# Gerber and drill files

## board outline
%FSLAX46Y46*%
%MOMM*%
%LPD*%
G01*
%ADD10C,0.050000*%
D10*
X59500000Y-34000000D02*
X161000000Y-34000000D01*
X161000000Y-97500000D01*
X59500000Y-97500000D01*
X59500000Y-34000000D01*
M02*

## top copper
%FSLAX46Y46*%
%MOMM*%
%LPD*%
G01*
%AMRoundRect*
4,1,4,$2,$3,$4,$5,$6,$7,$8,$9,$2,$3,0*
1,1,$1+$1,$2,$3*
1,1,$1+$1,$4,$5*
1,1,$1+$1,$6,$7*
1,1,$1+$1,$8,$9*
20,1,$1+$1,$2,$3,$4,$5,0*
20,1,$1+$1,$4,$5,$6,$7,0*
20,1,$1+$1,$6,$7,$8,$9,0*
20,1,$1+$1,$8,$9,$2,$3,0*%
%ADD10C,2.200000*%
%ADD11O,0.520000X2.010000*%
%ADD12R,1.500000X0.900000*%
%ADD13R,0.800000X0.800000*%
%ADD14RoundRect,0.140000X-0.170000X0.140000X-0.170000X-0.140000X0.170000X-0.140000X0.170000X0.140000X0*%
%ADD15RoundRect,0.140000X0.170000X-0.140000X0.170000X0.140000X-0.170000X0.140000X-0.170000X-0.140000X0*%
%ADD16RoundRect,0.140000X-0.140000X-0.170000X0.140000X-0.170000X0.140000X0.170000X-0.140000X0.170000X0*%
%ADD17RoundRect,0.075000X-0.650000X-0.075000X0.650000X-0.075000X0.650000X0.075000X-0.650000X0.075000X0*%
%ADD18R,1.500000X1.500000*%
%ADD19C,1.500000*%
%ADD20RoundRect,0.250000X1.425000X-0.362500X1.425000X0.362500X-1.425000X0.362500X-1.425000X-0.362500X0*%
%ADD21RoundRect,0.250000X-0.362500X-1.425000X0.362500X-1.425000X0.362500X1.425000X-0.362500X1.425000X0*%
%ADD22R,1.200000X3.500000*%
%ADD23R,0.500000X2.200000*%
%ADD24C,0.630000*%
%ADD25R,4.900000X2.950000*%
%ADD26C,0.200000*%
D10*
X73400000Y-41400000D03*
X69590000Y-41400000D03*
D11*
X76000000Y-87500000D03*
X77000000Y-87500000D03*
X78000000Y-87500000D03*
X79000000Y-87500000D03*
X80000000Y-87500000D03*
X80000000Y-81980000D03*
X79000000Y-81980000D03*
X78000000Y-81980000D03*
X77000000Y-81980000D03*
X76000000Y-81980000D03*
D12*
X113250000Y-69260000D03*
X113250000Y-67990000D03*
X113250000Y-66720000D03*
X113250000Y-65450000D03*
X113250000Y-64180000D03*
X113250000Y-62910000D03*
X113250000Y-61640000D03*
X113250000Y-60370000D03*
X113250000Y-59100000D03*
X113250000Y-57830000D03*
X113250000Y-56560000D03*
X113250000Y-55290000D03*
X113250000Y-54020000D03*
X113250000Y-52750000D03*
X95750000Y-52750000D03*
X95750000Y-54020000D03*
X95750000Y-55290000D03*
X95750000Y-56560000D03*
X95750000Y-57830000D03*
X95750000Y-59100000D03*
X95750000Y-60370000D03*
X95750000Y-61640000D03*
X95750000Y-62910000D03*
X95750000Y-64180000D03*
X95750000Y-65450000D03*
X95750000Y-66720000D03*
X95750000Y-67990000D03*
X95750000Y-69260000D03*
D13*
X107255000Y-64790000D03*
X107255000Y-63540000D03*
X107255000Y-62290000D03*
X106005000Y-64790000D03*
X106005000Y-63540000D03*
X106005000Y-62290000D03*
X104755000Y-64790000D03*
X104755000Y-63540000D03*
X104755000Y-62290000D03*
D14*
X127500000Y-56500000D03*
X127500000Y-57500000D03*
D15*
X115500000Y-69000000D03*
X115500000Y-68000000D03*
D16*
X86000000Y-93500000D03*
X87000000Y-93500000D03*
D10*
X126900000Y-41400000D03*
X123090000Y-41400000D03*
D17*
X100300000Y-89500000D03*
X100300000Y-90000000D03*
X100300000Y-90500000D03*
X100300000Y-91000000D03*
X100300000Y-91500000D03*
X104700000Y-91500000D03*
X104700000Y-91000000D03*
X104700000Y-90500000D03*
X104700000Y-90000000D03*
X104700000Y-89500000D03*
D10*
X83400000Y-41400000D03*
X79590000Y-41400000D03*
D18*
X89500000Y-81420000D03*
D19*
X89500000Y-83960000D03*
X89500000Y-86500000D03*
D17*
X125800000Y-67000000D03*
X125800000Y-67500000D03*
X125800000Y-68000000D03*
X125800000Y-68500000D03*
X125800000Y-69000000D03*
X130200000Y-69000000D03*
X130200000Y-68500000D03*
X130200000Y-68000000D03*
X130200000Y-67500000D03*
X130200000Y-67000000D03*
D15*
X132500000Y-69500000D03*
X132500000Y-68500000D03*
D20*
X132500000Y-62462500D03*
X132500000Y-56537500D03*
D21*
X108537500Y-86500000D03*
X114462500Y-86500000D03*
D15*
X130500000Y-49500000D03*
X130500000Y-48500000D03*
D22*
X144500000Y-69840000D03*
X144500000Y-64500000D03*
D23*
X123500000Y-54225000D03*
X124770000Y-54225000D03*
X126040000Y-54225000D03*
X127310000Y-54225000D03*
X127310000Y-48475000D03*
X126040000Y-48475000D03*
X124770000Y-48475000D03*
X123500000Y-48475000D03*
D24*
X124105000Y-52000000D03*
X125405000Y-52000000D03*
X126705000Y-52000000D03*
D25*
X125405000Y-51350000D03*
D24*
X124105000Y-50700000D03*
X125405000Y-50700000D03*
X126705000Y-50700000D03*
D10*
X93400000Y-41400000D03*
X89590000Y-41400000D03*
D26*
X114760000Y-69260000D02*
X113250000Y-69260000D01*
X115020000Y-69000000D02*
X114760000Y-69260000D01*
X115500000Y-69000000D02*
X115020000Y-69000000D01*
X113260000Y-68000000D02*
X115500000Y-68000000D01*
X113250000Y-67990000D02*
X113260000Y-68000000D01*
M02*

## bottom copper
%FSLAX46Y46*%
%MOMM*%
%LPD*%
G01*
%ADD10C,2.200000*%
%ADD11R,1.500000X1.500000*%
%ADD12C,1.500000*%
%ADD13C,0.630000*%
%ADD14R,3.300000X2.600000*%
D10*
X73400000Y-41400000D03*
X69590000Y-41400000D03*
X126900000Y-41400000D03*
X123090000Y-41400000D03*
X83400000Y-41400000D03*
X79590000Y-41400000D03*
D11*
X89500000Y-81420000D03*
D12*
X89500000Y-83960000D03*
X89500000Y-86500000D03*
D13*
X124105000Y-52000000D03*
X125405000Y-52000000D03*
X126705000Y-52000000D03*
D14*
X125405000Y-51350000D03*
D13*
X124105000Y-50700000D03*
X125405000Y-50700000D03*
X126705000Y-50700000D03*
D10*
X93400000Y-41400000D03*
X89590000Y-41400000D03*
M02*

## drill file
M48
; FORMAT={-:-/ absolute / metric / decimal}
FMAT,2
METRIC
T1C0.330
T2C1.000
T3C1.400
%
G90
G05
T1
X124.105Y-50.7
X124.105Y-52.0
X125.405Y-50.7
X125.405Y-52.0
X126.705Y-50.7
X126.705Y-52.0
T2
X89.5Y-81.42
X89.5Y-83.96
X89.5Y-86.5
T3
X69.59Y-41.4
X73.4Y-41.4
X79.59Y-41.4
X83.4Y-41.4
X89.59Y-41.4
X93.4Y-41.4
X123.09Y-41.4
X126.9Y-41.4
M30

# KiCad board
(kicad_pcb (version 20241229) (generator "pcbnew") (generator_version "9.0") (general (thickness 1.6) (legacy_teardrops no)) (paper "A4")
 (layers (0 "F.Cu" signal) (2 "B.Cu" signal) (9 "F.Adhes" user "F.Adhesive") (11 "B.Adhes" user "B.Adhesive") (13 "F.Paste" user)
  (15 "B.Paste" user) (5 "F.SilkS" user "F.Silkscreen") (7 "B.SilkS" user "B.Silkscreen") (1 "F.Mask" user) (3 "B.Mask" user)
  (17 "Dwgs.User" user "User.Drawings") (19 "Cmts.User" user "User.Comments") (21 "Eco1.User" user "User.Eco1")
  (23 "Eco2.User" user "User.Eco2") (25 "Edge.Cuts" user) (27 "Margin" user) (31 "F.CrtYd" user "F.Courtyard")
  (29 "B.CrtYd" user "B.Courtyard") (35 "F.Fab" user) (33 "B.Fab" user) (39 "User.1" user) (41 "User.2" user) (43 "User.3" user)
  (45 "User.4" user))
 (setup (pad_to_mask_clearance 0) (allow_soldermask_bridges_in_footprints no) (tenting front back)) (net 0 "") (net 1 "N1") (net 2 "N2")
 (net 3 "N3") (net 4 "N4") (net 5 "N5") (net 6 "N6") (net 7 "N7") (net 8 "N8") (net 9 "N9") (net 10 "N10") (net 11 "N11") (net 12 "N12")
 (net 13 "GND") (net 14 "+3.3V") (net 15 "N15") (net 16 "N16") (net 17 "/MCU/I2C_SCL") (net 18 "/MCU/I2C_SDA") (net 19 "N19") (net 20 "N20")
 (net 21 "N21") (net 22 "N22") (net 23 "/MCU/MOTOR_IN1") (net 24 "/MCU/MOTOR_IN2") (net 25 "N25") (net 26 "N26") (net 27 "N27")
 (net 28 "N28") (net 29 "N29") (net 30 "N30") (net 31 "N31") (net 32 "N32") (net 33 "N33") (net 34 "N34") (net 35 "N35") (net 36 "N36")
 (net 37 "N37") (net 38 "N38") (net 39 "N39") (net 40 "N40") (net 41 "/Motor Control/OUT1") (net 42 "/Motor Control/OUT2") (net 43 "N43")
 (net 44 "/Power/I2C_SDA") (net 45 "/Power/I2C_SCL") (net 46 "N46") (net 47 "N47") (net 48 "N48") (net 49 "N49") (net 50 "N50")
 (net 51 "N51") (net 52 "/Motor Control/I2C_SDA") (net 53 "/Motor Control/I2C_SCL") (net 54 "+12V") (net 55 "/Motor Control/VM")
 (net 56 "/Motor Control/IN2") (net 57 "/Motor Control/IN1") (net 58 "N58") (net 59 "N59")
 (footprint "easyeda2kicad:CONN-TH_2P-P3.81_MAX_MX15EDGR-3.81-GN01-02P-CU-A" (layer "F.Cu") (at 71.5 41.4 180)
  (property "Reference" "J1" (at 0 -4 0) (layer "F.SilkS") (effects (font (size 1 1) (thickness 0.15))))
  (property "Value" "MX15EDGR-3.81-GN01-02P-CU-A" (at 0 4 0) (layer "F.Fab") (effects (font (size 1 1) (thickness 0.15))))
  (pad "1" thru_hole circle (at -1.9 0 180) (size 2.2 2.2) (drill 1.399997) (layers "*.Cu" "*.Mask") (remove_unused_layers no) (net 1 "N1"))
  (pad "2" thru_hole circle (at 1.91 0 180) (size 2.2 2.2) (drill 1.399997) (layers "*.Cu" "*.Mask") (remove_unused_layers no) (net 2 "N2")))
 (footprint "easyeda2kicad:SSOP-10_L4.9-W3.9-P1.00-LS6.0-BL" (layer "F.Cu") (at 78 84.74)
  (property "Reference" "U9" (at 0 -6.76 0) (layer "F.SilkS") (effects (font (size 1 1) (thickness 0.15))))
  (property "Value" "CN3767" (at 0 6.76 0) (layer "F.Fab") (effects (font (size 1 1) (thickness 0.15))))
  (pad "1" smd oval (at -2 2.76) (size 0.52 2.01) (layers "F.Cu" "F.Mask" "F.Paste") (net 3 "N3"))
  (pad "2" smd oval (at -1 2.76) (size 0.52 2.01) (layers "F.Cu" "F.Mask" "F.Paste") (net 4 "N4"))
  (pad "3" smd oval (at 0 2.76) (size 0.52 2.01) (layers "F.Cu" "F.Mask" "F.Paste") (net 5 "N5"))
  (pad "4" smd oval (at 1 2.76) (size 0.52 2.01) (layers "F.Cu" "F.Mask" "F.Paste") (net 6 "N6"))
  (pad "5" smd oval (at 2 2.76) (size 0.52 2.01) (layers "F.Cu" "F.Mask" "F.Paste") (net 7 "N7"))
  (pad "6" smd oval (at 2 -2.76) (size 0.52 2.01) (layers "F.Cu" "F.Mask" "F.Paste") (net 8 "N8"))
  (pad "7" smd oval (at 1 -2.76) (size 0.52 2.01) (layers "F.Cu" "F.Mask" "F.Paste") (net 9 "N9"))
  (pad "8" smd oval (at 0 -2.76) (size 0.52 2.01) (layers "F.Cu" "F.Mask" "F.Paste") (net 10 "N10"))
  (pad "9" smd oval (at -1 -2.76) (size 0.52 2.01) (layers "F.Cu" "F.Mask" "F.Paste") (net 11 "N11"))
  (pad "10" smd oval (at -2 -2.76) (size 0.52 2.01) (layers "F.Cu" "F.Mask" "F.Paste") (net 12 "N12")))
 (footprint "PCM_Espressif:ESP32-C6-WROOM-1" (layer "F.Cu") (at 104.5 61 180)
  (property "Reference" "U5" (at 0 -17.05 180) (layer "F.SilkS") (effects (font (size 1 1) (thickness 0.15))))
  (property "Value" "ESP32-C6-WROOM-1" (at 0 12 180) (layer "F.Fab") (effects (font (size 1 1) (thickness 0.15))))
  (pad "1" smd rect (at -8.75 -8.26 180) (size 1.5 0.9) (layers "F.Cu" "F.Mask" "F.Paste") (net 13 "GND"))
  (pad "2" smd rect (at -8.75 -6.99 180) (size 1.5 0.9) (layers "F.Cu" "F.Mask" "F.Paste") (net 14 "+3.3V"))
  (pad "3" smd rect (at -8.75 -5.72 180) (size 1.5 0.9) (layers "F.Cu" "F.Mask" "F.Paste") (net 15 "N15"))
  (pad "4" smd rect (at -8.75 -4.45 180) (size 1.5 0.9) (layers "F.Cu" "F.Mask" "F.Paste") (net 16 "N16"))
  (pad "5" smd rect (at -8.75 -3.18 180) (size 1.5 0.9) (layers "F.Cu" "F.Mask" "F.Paste") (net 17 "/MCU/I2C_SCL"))
  (pad "6" smd rect (at -8.75 -1.91 180) (size 1.5 0.9) (layers "F.Cu" "F.Mask" "F.Paste") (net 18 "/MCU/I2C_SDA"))
  (pad "7" smd rect (at -8.75 -0.64 180) (size 1.5 0.9) (layers "F.Cu" "F.Mask" "F.Paste") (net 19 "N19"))
  (pad "8" smd rect (at -8.75 0.63 180) (size 1.5 0.9) (layers "F.Cu" "F.Mask" "F.Paste") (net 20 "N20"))
  (pad "9" smd rect (at -8.75 1.9 180) (size 1.5 0.9) (layers "F.Cu" "F.Mask" "F.Paste") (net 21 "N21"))
  (pad "10" smd rect (at -8.75 3.17 180) (size 1.5 0.9) (layers "F.Cu" "F.Mask" "F.Paste") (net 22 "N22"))
  (pad "11" smd rect (at -8.75 4.44 180) (size 1.5 0.9) (layers "F.Cu" "F.Mask" "F.Paste") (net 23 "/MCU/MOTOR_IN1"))
  (pad "12" smd rect (at -8.75 5.71 180) (size 1.5 0.9) (layers "F.Cu" "F.Mask" "F.Paste") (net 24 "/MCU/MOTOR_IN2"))
  (pad "13" smd rect (at -8.75 6.98 180) (size 1.5 0.9) (layers "F.Cu" "F.Mask" "F.Paste") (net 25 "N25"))
  (pad "14" smd rect (at -8.75 8.25 180) (size 1.5 0.9) (layers "F.Cu" "F.Mask" "F.Paste") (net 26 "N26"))
  (pad "15" smd rect (at 8.75 8.25) (size 1.5 0.9) (layers "F.Cu" "F.Mask" "F.Paste") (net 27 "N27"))
  (pad "16" smd rect (at 8.75 6.98) (size 1.5 0.9) (layers "F.Cu" "F.Mask" "F.Paste") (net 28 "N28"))
  (pad "17" smd rect (at 8.75 5.71) (size 1.5 0.9) (layers "F.Cu" "F.Mask" "F.Paste") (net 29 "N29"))
  (pad "18" smd rect (at 8.75 4.44) (size 1.5 0.9) (layers "F.Cu" "F.Mask" "F.Paste") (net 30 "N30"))
  (pad "19" smd rect (at 8.75 3.17) (size 1.5 0.9) (layers "F.Cu" "F.Mask" "F.Paste") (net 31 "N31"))
  (pad "20" smd rect (at 8.75 1.9) (size 1.5 0.9) (layers "F.Cu" "F.Mask" "F.Paste") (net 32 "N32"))
  (pad "21" smd rect (at 8.75 0.63) (size 1.5 0.9) (layers "F.Cu" "F.Mask" "F.Paste") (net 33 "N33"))
  (pad "22" smd rect (at 8.75 -0.64) (size 1.5 0.9) (layers "F.Cu" "F.Mask" "F.Paste") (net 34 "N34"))
  (pad "23" smd rect (at 8.75 -1.91) (size 1.5 0.9) (layers "F.Cu" "F.Mask" "F.Paste") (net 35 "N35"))
  (pad "24" smd rect (at 8.75 -3.18) (size 1.5 0.9) (layers "F.Cu" "F.Mask" "F.Paste") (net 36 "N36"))
  (pad "25" smd rect (at 8.75 -4.45) (size 1.5 0.9) (layers "F.Cu" "F.Mask" "F.Paste") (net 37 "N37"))
  (pad "26" smd rect (at 8.75 -5.72) (size 1.5 0.9) (layers "F.Cu" "F.Mask" "F.Paste") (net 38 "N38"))
  (pad "27" smd rect (at 8.75 -6.99) (size 1.5 0.9) (layers "F.Cu" "F.Mask" "F.Paste") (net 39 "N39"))
  (pad "28" smd rect (at 8.75 -8.26) (size 1.5 0.9) (layers "F.Cu" "F.Mask" "F.Paste") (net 13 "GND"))
  (pad "29" smd rect (at -2.755 -3.79) (size 0.8 0.8) (layers "F.Cu" "F.Mask" "F.Paste") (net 13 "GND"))
  (pad "29" smd rect (at -2.755 -2.54) (size 0.8 0.8) (layers "F.Cu" "F.Mask" "F.Paste") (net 13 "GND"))
  (pad "29" smd rect (at -2.755 -1.29) (size 0.8 0.8) (layers "F.Cu" "F.Mask" "F.Paste") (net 13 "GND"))
  (pad "29" smd rect (at -1.505 -3.79) (size 0.8 0.8) (layers "F.Cu" "F.Mask" "F.Paste") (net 13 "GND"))
  (pad "29" smd rect (at -1.505 -2.54) (size 0.8 0.8) (layers "F.Cu" "F.Mask" "F.Paste") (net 13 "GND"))
  (pad "29" smd rect (at -1.505 -1.29) (size 0.8 0.8) (layers "F.Cu" "F.Mask" "F.Paste") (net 13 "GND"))
  (pad "29" smd rect (at -0.255 -3.79) (size 0.8 0.8) (layers "F.Cu" "F.Mask" "F.Paste") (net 13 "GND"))
  (pad "29" smd rect (at -0.255 -2.54) (size 0.8 0.8) (layers "F.Cu" "F.Mask" "F.Paste") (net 13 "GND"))
  (pad "29" smd rect (at -0.255 -1.29) (size 0.8 0.8) (layers "F.Cu" "F.Mask" "F.Paste") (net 13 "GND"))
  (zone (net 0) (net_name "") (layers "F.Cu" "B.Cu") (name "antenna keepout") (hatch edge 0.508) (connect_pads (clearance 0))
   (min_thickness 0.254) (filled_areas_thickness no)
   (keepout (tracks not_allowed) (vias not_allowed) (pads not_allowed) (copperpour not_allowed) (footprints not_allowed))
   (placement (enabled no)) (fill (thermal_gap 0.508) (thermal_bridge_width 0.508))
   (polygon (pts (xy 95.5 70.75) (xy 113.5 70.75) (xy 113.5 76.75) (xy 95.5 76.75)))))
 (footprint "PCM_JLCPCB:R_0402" (layer "F.Cu") (at 127.5 57 -90)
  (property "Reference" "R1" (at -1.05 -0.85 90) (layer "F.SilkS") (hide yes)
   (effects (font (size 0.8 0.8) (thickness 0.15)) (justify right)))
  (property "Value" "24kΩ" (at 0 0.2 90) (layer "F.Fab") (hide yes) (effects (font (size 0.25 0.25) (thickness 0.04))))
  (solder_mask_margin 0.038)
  (pad "1" smd roundrect (at -0.5 0 270) (size 0.56 0.62) (layers "F.Cu" "F.Mask" "F.Paste") (roundrect_rratio 0.25) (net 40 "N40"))
  (pad "2" smd roundrect (at 0.5 0 270) (size 0.56 0.62) (layers "F.Cu" "F.Mask" "F.Paste") (roundrect_rratio 0.25) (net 13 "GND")))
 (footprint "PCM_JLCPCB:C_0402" (layer "F.Cu") (at 115.5 68.5 90)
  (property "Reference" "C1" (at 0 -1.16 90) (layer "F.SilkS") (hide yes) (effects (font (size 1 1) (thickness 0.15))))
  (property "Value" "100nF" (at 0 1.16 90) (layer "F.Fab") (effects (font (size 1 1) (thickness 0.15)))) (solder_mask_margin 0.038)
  (pad "1" smd roundrect (at -0.5 0 90) (size 0.56 0.62) (layers "F.Cu" "F.Mask" "F.Paste") (roundrect_rratio 0.25) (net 13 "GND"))
  (pad "2" smd roundrect (at 0.5 0 90) (size 0.56 0.62) (layers "F.Cu" "F.Mask" "F.Paste") (roundrect_rratio 0.25) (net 14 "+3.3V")))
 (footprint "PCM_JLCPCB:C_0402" (layer "F.Cu") (at 86.5 93.5)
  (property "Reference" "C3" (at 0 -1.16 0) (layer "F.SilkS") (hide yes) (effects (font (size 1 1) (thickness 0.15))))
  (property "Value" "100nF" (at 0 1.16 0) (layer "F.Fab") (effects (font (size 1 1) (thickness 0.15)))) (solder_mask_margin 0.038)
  (pad "1" smd roundrect (at -0.5 0) (size 0.56 0.62) (layers "F.Cu" "F.Mask" "F.Paste") (roundrect_rratio 0.25) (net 14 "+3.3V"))
  (pad "2" smd roundrect (at 0.5 0) (size 0.56 0.62) (layers "F.Cu" "F.Mask" "F.Paste") (roundrect_rratio 0.25) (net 13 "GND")))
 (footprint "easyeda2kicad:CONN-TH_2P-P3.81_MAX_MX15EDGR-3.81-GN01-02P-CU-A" (layer "F.Cu") (at 125 41.4 180)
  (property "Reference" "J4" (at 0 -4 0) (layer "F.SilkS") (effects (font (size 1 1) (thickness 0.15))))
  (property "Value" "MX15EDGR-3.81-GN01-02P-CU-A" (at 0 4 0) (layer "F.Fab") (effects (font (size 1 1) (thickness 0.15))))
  (pad "1" thru_hole circle (at -1.9 0 180) (size 2.2 2.2) (drill 1.399997) (layers "*.Cu" "*.Mask") (remove_unused_layers no)
   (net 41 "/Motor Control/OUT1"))
  (pad "2" thru_hole circle (at 1.91 0 180) (size 2.2 2.2) (drill 1.399997) (layers "*.Cu" "*.Mask") (remove_unused_layers no)
   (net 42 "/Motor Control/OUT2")))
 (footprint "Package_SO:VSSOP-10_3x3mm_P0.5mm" (layer "F.Cu") (at 102.5 90.5)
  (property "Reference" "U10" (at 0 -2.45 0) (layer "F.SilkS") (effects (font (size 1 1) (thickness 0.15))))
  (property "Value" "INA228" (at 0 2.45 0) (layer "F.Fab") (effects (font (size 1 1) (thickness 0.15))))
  (pad "1" smd roundrect (at -2.2 -1) (size 1.45 0.3) (layers "F.Cu" "F.Mask" "F.Paste") (roundrect_rratio 0.25) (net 13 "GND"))
  (pad "2" smd roundrect (at -2.2 -0.5) (size 1.45 0.3) (layers "F.Cu" "F.Mask" "F.Paste") (roundrect_rratio 0.25) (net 13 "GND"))
  (pad "3" smd roundrect (at -2.2 0) (size 1.45 0.3) (layers "F.Cu" "F.Mask" "F.Paste") (roundrect_rratio 0.25) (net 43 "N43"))
  (pad "4" smd roundrect (at -2.2 0.5) (size 1.45 0.3) (layers "F.Cu" "F.Mask" "F.Paste") (roundrect_rratio 0.25) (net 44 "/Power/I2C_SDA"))
  (pad "5" smd roundrect (at -2.2 1) (size 1.45 0.3) (layers "F.Cu" "F.Mask" "F.Paste") (roundrect_rratio 0.25) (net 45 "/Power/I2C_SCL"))
  (pad "6" smd roundrect (at 2.2 1) (size 1.45 0.3) (layers "F.Cu" "F.Mask" "F.Paste") (roundrect_rratio 0.25) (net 14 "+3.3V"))
  (pad "7" smd roundrect (at 2.2 0.5) (size 1.45 0.3) (layers "F.Cu" "F.Mask" "F.Paste") (roundrect_rratio 0.25) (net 13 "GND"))
  (pad "8" smd roundrect (at 2.2 0) (size 1.45 0.3) (layers "F.Cu" "F.Mask" "F.Paste") (roundrect_rratio 0.25) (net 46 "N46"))
  (pad "9" smd roundrect (at 2.2 -0.5) (size 1.45 0.3) (layers "F.Cu" "F.Mask" "F.Paste") (roundrect_rratio 0.25) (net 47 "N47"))
  (pad "10" smd roundrect (at 2.2 -1) (size 1.45 0.3) (layers "F.Cu" "F.Mask" "F.Paste") (roundrect_rratio 0.25) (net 46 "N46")))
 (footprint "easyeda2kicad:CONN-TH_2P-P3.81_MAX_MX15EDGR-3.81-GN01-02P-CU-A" (layer "F.Cu") (at 81.5 41.4 180)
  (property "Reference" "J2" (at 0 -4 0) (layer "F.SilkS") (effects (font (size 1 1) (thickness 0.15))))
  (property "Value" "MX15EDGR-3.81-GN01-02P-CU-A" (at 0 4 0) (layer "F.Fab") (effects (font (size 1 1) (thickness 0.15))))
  (pad "1" thru_hole circle (at -1.9 0 180) (size 2.2 2.2) (drill 1.399997) (layers "*.Cu" "*.Mask") (remove_unused_layers no)
   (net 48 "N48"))
  (pad "2" thru_hole circle (at 1.91 0 180) (size 2.2 2.2) (drill 1.399997) (layers "*.Cu" "*.Mask") (remove_unused_layers no)
   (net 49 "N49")))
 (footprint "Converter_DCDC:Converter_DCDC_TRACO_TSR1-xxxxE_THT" (layer "F.Cu") (at 89.5 81.42)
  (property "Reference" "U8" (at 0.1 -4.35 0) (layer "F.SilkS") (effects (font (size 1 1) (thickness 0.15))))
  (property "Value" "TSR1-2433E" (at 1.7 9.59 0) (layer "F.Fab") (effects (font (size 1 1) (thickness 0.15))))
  (pad "1" thru_hole rect (at 0 0) (size 1.5 1.5) (drill 1) (layers "*.Cu" "*.Mask") (remove_unused_layers no) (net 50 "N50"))
  (pad "2" thru_hole circle (at 0 2.54) (size 1.5 1.5) (drill 1) (layers "*.Cu" "*.Mask") (remove_unused_layers no) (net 13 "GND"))
  (pad "3" thru_hole circle (at 0 5.08) (size 1.5 1.5) (drill 1) (layers "*.Cu" "*.Mask") (remove_unused_layers no) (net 14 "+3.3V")))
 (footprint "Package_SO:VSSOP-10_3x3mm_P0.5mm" (layer "F.Cu") (at 128 68)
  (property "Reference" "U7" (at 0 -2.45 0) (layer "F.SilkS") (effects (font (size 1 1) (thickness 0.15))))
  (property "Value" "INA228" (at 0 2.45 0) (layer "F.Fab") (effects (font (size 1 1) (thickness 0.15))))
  (pad "1" smd roundrect (at -2.2 -1) (size 1.45 0.3) (layers "F.Cu" "F.Mask" "F.Paste") (roundrect_rratio 0.25) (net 13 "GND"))
  (pad "2" smd roundrect (at -2.2 -0.5) (size 1.45 0.3) (layers "F.Cu" "F.Mask" "F.Paste") (roundrect_rratio 0.25) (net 13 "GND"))
  (pad "3" smd roundrect (at -2.2 0) (size 1.45 0.3) (layers "F.Cu" "F.Mask" "F.Paste") (roundrect_rratio 0.25) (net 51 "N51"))
  (pad "4" smd roundrect (at -2.2 0.5) (size 1.45 0.3) (layers "F.Cu" "F.Mask" "F.Paste") (roundrect_rratio 0.25)
   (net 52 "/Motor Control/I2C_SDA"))
  (pad "5" smd roundrect (at -2.2 1) (size 1.45 0.3) (layers "F.Cu" "F.Mask" "F.Paste") (roundrect_rratio 0.25)
   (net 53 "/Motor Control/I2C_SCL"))
  (pad "6" smd roundrect (at 2.2 1) (size 1.45 0.3) (layers "F.Cu" "F.Mask" "F.Paste") (roundrect_rratio 0.25) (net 14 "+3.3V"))
  (pad "7" smd roundrect (at 2.2 0.5) (size 1.45 0.3) (layers "F.Cu" "F.Mask" "F.Paste") (roundrect_rratio 0.25) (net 13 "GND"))
  (pad "8" smd roundrect (at 2.2 0) (size 1.45 0.3) (layers "F.Cu" "F.Mask" "F.Paste") (roundrect_rratio 0.25) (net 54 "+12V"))
  (pad "9" smd roundrect (at 2.2 -0.5) (size 1.45 0.3) (layers "F.Cu" "F.Mask" "F.Paste") (roundrect_rratio 0.25)
   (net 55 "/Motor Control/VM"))
  (pad "10" smd roundrect (at 2.2 -1) (size 1.45 0.3) (layers "F.Cu" "F.Mask" "F.Paste") (roundrect_rratio 0.25) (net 54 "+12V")))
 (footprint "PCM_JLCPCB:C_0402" (layer "F.Cu") (at 132.5 69 90)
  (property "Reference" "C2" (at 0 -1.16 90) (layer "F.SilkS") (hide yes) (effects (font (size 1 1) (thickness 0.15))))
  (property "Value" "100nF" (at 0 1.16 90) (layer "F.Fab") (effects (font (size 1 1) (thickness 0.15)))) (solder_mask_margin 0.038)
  (pad "1" smd roundrect (at -0.5 0 90) (size 0.56 0.62) (layers "F.Cu" "F.Mask" "F.Paste") (roundrect_rratio 0.25) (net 14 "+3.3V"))
  (pad "2" smd roundrect (at 0.5 0 90) (size 0.56 0.62) (layers "F.Cu" "F.Mask" "F.Paste") (roundrect_rratio 0.25) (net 13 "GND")))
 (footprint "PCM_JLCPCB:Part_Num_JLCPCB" (layer "F.Cu") (at 64 88.5 90)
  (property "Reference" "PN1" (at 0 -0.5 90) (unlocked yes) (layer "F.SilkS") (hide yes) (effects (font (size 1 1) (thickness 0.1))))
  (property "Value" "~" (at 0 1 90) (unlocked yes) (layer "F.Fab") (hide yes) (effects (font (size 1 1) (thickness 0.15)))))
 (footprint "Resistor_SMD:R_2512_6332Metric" (layer "F.Cu") (at 132.5 59.5 90)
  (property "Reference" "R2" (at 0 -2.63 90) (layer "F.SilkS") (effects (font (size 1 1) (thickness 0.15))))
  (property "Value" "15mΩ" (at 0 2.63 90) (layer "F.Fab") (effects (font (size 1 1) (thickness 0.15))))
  (pad "1" smd roundrect (at -2.9625 0 90) (size 1.225 3.35) (layers "F.Cu" "F.Mask" "F.Paste") (roundrect_rratio 0.204082) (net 54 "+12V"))
  (pad "2" smd roundrect (at 2.9625 0 90) (size 1.225 3.35) (layers "F.Cu" "F.Mask" "F.Paste") (roundrect_rratio 0.204082)
   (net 55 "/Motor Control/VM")))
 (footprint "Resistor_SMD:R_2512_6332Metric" (layer "F.Cu") (at 111.5 86.5)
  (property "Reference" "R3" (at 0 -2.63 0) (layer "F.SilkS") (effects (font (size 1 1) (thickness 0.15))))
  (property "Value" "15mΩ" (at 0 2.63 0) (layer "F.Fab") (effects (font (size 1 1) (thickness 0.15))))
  (pad "1" smd roundrect (at -2.9625 0) (size 1.225 3.35) (layers "F.Cu" "F.Mask" "F.Paste") (roundrect_rratio 0.204082) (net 46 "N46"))
  (pad "2" smd roundrect (at 2.9625 0) (size 1.225 3.35) (layers "F.Cu" "F.Mask" "F.Paste") (roundrect_rratio 0.204082) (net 47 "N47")))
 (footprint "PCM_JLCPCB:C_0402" (layer "F.Cu") (at 130.5 49 90)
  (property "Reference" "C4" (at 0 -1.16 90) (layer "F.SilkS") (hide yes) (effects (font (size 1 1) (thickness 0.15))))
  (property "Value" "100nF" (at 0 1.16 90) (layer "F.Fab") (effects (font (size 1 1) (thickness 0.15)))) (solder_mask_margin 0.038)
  (pad "1" smd roundrect (at -0.5 0 90) (size 0.56 0.62) (layers "F.Cu" "F.Mask" "F.Paste") (roundrect_rratio 0.25) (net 13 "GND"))
  (pad "2" smd roundrect (at 0.5 0 90) (size 0.56 0.62) (layers "F.Cu" "F.Mask" "F.Paste") (roundrect_rratio 0.25)
   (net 55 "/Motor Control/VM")))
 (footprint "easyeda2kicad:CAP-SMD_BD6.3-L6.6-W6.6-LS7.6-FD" (layer "F.Cu") (at 144.5 67.17 90)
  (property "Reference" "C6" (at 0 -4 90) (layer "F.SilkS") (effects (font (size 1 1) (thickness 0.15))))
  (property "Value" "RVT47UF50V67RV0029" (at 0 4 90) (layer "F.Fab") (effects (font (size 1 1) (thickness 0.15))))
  (pad "1" smd rect (at -2.67 0 90) (size 3.5 1.2) (layers "F.Cu" "F.Mask" "F.Paste") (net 13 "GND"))
  (pad "2" smd rect (at 2.67 0 90) (size 3.5 1.2) (layers "F.Cu" "F.Mask" "F.Paste") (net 54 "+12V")))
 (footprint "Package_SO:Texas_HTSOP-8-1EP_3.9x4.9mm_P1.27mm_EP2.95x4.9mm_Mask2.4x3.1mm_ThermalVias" (layer "F.Cu") (at 125.405 51.35 90)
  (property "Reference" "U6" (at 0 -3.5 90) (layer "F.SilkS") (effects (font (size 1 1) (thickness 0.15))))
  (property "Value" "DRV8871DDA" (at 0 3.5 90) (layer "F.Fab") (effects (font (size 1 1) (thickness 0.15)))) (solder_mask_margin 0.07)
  (pad "" smd rect (at 0 0 90) (size 2.4 3.1) (layers "F.Mask"))
  (pad "" smd rect (at 0 0 90) (size 2.4 3.1) (layers "F.Paste"))
  (pad "1" smd rect (at -2.875 -1.905 90) (size 2.2 0.5) (layers "F.Cu" "F.Mask" "F.Paste") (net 13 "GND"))
  (pad "2" smd rect (at -2.875 -0.635 90) (size 2.2 0.5) (layers "F.Cu" "F.Mask" "F.Paste") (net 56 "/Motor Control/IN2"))
  (pad "3" smd rect (at -2.875 0.635 90) (size 2.2 0.5) (layers "F.Cu" "F.Mask" "F.Paste") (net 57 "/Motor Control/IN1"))
  (pad "4" smd rect (at -2.875 1.905 90) (size 2.2 0.5) (layers "F.Cu" "F.Mask" "F.Paste") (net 40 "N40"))
  (pad "5" smd rect (at 2.875 1.905 90) (size 2.2 0.5) (layers "F.Cu" "F.Mask" "F.Paste") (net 55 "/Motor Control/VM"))
  (pad "6" smd rect (at 2.875 0.635 90) (size 2.2 0.5) (layers "F.Cu" "F.Mask" "F.Paste") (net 41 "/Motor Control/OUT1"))
  (pad "7" smd rect (at 2.875 -0.635 90) (size 2.2 0.5) (layers "F.Cu" "F.Mask" "F.Paste") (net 13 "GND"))
  (pad "8" smd rect (at 2.875 -1.905 90) (size 2.2 0.5) (layers "F.Cu" "F.Mask" "F.Paste") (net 42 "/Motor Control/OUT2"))
  (pad "9" thru_hole circle (at -0.65 -1.3 90) (size 0.63 0.63) (drill 0.33) (layers "*.Cu" "*.Mask") (remove_unused_layers no)
   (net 13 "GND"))
  (pad "9" thru_hole circle (at -0.65 0 90) (size 0.63 0.63) (drill 0.33) (layers "*.Cu" "*.Mask") (remove_unused_layers no) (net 13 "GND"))
  (pad "9" thru_hole circle (at -0.65 1.3 90) (size 0.63 0.63) (drill 0.33) (layers "*.Cu" "*.Mask") (remove_unused_layers no)
   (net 13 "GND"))
  (pad "9" smd rect (at 0 0 90) (size 2.6 3.3) (layers "B.Cu") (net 13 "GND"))
  (pad "9" smd rect (at 0 0 90) (size 2.95 4.9) (layers "F.Cu") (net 13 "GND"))
  (pad "9" thru_hole circle (at 0.65 -1.3 90) (size 0.63 0.63) (drill 0.33) (layers "*.Cu" "*.Mask") (remove_unused_layers no)
   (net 13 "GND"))
  (pad "9" thru_hole circle (at 0.65 0 90) (size 0.63 0.63) (drill 0.33) (layers "*.Cu" "*.Mask") (remove_unused_layers no) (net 13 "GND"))
  (pad "9" thru_hole circle (at 0.65 1.3 90) (size 0.63 0.63) (drill 0.33) (layers "*.Cu" "*.Mask") (remove_unused_layers no) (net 13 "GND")))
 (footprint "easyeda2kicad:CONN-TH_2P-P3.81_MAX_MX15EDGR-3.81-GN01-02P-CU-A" (layer "F.Cu") (at 91.5 41.4 180)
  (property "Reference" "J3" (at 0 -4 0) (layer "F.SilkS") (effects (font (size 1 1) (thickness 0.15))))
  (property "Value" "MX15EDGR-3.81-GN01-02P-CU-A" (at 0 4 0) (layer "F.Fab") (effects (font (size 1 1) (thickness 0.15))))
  (pad "1" thru_hole circle (at -1.9 0 180) (size 2.2 2.2) (drill 1.399997) (layers "*.Cu" "*.Mask") (remove_unused_layers no)
   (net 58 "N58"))
  (pad "2" thru_hole circle (at 1.91 0 180) (size 2.2 2.2) (drill 1.399997) (layers "*.Cu" "*.Mask") (remove_unused_layers no)
   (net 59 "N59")))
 (gr_rect (start 59.5 34) (end 161 97.5) (stroke (width 0.05) (type default)) (fill no) (layer "Edge.Cuts"))
 (segment (start 114.76 69.26) (end 113.25 69.26) (width 0.2) (layer "F.Cu") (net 13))
 (segment (start 115.02 69) (end 114.76 69.26) (width 0.2) (layer "F.Cu") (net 13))
 (segment (start 115.5 69) (end 115.02 69) (width 0.2) (layer "F.Cu") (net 13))
 (segment (start 113.26 68) (end 115.5 68) (width 0.2) (layer "F.Cu") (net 14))
 (segment (start 113.25 67.99) (end 113.26 68) (width 0.2) (layer "F.Cu") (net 14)))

